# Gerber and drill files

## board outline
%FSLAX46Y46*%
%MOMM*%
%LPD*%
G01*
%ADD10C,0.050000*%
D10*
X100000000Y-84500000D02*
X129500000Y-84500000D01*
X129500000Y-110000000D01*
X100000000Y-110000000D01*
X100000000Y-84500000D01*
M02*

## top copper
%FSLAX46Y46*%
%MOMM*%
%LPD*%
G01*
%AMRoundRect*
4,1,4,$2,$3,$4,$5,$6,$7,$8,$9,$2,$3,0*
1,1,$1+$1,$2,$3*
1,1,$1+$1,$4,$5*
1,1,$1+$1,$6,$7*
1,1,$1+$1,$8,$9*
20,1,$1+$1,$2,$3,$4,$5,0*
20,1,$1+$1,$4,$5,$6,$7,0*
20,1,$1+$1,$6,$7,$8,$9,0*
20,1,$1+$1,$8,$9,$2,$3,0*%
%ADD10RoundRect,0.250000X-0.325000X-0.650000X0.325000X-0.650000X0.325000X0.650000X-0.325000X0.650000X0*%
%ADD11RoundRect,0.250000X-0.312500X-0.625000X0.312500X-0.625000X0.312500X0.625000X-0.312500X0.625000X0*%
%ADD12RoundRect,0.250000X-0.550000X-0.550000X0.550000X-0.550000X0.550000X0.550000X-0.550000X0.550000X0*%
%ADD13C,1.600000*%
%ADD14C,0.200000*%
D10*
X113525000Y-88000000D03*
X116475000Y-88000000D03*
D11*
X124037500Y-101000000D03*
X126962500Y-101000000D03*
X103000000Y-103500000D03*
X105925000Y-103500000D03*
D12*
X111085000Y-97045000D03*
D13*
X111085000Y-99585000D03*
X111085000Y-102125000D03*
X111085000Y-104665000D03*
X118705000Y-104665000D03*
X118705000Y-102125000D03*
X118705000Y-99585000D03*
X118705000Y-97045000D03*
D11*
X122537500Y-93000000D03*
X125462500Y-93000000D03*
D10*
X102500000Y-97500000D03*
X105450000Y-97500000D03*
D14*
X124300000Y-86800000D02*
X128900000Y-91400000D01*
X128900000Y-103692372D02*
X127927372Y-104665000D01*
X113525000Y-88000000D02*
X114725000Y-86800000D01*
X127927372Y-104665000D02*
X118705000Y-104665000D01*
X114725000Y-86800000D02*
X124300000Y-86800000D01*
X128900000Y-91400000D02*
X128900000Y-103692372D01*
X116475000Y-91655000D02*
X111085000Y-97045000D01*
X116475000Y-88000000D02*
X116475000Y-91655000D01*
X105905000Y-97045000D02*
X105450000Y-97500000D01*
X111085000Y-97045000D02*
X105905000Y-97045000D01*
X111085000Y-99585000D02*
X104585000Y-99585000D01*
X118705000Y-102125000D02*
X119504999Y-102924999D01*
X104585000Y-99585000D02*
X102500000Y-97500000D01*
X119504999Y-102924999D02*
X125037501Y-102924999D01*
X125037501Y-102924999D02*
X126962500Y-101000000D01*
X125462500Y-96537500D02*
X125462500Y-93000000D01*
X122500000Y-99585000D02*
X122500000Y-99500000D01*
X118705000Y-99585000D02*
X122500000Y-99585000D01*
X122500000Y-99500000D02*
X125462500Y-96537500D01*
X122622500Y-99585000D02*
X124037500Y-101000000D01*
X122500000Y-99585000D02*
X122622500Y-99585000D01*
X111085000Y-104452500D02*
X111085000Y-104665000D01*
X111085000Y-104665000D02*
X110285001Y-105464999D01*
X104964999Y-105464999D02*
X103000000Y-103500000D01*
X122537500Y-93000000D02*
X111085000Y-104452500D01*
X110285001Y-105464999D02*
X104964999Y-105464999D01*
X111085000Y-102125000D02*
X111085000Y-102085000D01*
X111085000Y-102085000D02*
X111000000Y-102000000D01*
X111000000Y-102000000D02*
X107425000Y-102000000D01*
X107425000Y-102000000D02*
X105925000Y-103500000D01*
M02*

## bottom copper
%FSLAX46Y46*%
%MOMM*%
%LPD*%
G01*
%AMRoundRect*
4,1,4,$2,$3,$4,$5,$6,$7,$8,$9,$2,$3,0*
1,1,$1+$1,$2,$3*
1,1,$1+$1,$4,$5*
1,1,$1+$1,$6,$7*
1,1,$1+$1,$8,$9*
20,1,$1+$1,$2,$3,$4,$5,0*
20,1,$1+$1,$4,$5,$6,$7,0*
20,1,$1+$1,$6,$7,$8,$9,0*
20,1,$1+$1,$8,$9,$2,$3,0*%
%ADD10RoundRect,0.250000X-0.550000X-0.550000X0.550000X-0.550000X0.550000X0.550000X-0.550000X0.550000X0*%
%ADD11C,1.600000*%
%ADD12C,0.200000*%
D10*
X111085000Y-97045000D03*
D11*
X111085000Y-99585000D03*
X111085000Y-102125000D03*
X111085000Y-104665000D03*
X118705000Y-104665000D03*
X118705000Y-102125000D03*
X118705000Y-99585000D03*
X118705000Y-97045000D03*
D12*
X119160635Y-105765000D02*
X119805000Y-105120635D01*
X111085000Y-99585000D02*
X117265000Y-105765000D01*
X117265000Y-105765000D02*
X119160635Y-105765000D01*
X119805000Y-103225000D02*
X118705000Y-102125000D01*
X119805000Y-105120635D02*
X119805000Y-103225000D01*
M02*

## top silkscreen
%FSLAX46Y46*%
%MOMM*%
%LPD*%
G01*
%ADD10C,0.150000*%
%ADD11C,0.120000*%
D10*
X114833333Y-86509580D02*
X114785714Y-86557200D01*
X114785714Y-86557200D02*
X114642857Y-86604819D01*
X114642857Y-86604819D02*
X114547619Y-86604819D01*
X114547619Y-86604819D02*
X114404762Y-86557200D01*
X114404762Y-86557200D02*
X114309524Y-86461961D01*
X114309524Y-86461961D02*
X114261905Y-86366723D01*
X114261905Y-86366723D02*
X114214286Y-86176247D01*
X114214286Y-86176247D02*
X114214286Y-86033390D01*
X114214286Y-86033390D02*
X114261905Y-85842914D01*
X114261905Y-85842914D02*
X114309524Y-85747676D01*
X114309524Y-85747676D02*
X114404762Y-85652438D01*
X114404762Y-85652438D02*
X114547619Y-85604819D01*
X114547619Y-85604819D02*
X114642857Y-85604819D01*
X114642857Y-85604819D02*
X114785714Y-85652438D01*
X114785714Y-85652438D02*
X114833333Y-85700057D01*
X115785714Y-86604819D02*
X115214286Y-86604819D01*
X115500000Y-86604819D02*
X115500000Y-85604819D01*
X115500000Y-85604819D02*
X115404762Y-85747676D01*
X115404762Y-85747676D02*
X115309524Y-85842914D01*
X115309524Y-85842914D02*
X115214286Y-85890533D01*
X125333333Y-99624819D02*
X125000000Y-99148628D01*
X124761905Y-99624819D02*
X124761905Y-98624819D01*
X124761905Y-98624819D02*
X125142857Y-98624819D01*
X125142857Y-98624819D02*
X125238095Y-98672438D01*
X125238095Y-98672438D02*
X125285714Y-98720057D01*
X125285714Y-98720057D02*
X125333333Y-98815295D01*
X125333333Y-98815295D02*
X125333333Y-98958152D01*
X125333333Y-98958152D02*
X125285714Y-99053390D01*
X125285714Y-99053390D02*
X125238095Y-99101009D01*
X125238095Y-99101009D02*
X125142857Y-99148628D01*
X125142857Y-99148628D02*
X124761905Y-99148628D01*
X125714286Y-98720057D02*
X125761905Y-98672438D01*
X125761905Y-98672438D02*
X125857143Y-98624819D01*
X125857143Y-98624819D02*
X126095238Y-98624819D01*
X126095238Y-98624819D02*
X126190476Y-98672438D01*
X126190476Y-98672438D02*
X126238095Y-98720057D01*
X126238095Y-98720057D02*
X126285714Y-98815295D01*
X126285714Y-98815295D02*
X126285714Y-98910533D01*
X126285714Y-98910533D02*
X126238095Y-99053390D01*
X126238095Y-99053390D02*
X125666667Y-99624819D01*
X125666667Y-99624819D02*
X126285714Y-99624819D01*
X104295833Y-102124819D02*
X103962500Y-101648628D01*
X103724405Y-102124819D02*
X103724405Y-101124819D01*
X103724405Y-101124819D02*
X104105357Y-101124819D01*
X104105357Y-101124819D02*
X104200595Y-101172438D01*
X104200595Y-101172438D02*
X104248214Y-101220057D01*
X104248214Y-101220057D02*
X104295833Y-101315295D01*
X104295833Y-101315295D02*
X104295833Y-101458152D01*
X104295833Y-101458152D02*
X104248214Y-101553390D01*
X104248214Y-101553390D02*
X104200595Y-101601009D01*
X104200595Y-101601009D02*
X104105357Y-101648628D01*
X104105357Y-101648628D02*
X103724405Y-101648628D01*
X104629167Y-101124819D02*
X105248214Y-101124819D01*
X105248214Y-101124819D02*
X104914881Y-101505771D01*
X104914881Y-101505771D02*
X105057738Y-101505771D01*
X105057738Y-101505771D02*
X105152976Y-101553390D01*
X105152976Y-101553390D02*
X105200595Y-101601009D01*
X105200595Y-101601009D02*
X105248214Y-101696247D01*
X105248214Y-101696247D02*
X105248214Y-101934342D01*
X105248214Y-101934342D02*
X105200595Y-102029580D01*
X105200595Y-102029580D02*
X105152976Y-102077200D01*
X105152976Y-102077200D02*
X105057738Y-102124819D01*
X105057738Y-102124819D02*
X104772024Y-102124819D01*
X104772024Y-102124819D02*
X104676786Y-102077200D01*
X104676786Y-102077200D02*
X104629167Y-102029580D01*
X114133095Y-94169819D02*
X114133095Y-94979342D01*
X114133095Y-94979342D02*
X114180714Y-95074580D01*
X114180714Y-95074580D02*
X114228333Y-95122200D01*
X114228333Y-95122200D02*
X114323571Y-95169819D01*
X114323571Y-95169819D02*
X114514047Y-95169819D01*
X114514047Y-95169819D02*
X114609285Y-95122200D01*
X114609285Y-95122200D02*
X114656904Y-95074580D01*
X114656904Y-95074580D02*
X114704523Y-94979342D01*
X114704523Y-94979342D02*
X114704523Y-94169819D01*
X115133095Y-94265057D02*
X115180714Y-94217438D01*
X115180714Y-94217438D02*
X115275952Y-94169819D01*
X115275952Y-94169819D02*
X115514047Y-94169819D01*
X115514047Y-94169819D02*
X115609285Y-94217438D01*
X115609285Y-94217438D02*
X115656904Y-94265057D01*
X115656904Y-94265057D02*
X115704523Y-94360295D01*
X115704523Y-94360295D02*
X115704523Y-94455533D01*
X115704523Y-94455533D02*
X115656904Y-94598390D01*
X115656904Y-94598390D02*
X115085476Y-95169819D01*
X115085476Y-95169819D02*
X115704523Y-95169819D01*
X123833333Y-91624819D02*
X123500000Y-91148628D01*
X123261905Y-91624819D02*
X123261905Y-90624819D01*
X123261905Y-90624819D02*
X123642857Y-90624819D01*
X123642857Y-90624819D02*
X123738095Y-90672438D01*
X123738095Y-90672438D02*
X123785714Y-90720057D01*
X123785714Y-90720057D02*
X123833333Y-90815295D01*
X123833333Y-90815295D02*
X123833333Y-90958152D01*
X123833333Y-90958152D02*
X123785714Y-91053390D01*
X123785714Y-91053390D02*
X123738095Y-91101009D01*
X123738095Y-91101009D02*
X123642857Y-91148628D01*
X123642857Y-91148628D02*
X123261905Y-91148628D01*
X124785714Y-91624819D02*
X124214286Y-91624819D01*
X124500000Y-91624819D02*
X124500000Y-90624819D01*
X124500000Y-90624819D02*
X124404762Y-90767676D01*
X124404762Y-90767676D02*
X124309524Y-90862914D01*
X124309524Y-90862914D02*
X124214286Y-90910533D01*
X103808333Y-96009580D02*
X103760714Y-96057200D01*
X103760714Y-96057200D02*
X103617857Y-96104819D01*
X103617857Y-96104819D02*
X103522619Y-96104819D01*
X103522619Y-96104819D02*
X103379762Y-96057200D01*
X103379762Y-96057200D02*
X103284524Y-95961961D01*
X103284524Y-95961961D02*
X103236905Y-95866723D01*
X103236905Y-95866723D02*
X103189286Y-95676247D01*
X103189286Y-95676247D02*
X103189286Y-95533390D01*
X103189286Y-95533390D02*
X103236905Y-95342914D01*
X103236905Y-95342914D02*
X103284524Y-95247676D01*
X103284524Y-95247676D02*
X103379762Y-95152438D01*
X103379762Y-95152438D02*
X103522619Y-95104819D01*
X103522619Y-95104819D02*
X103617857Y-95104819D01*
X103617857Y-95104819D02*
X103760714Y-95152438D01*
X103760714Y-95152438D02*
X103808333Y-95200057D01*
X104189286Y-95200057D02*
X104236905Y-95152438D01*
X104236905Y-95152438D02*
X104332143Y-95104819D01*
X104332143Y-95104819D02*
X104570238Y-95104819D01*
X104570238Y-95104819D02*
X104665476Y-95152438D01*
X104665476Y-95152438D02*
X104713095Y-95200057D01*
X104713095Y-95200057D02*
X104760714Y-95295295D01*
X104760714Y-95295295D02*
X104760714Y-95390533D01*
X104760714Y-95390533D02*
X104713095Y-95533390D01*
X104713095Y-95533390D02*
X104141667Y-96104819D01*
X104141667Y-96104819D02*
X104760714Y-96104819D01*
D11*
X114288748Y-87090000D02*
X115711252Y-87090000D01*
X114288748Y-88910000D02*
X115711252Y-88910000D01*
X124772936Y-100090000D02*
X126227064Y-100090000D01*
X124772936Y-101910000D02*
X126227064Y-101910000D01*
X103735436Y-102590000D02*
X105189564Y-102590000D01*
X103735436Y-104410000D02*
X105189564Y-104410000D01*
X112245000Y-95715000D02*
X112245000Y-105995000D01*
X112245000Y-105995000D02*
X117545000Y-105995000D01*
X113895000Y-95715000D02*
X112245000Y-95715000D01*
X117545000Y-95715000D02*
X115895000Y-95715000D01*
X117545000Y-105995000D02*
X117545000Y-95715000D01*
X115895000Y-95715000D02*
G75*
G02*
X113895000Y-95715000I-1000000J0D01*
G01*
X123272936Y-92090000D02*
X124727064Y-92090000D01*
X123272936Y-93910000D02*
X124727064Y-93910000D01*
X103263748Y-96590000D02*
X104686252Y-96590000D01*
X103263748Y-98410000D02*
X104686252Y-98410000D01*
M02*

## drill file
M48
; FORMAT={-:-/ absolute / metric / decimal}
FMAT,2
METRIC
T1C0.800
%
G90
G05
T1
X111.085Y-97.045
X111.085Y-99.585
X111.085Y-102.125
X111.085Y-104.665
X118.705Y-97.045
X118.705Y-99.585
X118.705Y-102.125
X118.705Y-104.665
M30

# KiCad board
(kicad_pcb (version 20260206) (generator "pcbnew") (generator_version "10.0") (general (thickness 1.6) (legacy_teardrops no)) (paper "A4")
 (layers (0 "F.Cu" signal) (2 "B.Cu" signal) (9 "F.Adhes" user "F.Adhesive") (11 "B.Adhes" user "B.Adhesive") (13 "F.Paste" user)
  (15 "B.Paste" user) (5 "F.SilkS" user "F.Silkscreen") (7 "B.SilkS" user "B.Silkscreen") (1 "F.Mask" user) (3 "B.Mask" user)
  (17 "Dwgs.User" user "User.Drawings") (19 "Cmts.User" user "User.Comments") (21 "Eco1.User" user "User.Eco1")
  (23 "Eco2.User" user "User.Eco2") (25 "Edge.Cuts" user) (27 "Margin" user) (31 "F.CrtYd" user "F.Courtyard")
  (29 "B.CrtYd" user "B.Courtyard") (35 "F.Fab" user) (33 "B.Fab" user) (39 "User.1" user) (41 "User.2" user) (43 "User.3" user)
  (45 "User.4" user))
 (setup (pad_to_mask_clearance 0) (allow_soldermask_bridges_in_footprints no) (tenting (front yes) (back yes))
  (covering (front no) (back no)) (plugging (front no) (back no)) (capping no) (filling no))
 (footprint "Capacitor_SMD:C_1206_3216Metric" (layer "F.Cu") (at 115 88)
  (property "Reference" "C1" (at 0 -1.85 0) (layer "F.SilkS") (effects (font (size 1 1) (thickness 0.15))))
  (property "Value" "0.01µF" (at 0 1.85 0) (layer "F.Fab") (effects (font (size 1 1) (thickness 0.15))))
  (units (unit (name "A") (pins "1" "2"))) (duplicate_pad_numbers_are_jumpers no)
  (fp_line (start -0.711252 -0.91) (end 0.711252 -0.91) (stroke (width 0.12) (type solid)) (layer "F.SilkS"))
  (fp_line (start -0.711252 0.91) (end 0.711252 0.91) (stroke (width 0.12) (type solid)) (layer "F.SilkS"))
  (pad "1" smd roundrect (at -1.475 0) (size 1.15 1.8) (layers "F.Cu" "F.Mask" "F.Paste") (roundrect_rratio 0.217391) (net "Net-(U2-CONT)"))
  (pad "2" smd roundrect (at 1.475 0) (size 1.15 1.8) (layers "F.Cu" "F.Mask" "F.Paste") (roundrect_rratio 0.217391) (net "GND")))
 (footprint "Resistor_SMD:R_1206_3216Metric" (layer "F.Cu") (at 125.5 101)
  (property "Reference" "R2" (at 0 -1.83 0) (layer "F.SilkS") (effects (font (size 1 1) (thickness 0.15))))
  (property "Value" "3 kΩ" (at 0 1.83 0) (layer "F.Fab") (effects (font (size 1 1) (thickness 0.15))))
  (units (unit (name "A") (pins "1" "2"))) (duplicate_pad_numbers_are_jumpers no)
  (fp_line (start -0.727064 -0.91) (end 0.727064 -0.91) (stroke (width 0.12) (type solid)) (layer "F.SilkS"))
  (fp_line (start -0.727064 0.91) (end 0.727064 0.91) (stroke (width 0.12) (type solid)) (layer "F.SilkS"))
  (pad "1" smd roundrect (at -1.4625 0) (size 1.125 1.75) (layers "F.Cu" "F.Mask" "F.Paste") (roundrect_rratio 0.222222)
   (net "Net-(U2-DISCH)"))
  (pad "2" smd roundrect (at 1.4625 0) (size 1.125 1.75) (layers "F.Cu" "F.Mask" "F.Paste") (roundrect_rratio 0.222222)
   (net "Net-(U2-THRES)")))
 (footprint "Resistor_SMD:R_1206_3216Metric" (layer "F.Cu") (at 104.4625 103.5)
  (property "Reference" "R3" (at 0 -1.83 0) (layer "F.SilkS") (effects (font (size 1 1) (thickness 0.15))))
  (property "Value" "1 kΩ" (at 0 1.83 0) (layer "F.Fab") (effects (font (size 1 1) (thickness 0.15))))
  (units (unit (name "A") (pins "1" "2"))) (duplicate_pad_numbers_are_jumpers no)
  (fp_line (start -0.727064 -0.91) (end 0.727064 -0.91) (stroke (width 0.12) (type solid)) (layer "F.SilkS"))
  (fp_line (start -0.727064 0.91) (end 0.727064 0.91) (stroke (width 0.12) (type solid)) (layer "F.SilkS"))
  (pad "1" smd roundrect (at -1.4625 0) (size 1.125 1.75) (layers "F.Cu" "F.Mask" "F.Paste") (roundrect_rratio 0.222222)
   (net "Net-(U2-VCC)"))
  (pad "2" smd roundrect (at 1.4625 0) (size 1.125 1.75) (layers "F.Cu" "F.Mask" "F.Paste") (roundrect_rratio 0.222222) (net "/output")))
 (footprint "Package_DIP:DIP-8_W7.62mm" (layer "F.Cu") (at 111.085 97.045)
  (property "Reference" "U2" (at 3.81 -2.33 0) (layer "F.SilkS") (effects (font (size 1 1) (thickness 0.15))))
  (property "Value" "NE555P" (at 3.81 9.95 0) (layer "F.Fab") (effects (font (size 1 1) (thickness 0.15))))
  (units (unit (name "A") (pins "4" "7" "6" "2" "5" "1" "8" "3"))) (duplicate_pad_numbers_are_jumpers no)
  (fp_line (start 1.16 -1.33) (end 1.16 8.95) (stroke (width 0.12) (type solid)) (layer "F.SilkS"))
  (fp_line (start 1.16 8.95) (end 6.46 8.95) (stroke (width 0.12) (type solid)) (layer "F.SilkS"))
  (fp_line (start 2.81 -1.33) (end 1.16 -1.33) (stroke (width 0.12) (type solid)) (layer "F.SilkS"))
  (fp_line (start 6.46 -1.33) (end 4.81 -1.33) (stroke (width 0.12) (type solid)) (layer "F.SilkS"))
  (fp_line (start 6.46 8.95) (end 6.46 -1.33) (stroke (width 0.12) (type solid)) (layer "F.SilkS"))
  (fp_arc (start 4.81 -1.33) (mid 3.81 -0.33) (end 2.81 -1.33) (stroke (width 0.12) (type solid)) (layer "F.SilkS"))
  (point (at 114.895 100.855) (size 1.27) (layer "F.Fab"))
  (pad "1" thru_hole roundrect (at 0 0) (size 1.6 1.6) (drill 0.8) (layers "*.Cu" "*.Mask") (remove_unused_layers no)
   (roundrect_rratio 0.15625) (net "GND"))
  (pad "2" thru_hole circle (at 0 2.54) (size 1.6 1.6) (drill 0.8) (layers "*.Cu" "*.Mask") (remove_unused_layers no) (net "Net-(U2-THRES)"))
  (pad "3" thru_hole circle (at 0 5.08) (size 1.6 1.6) (drill 0.8) (layers "*.Cu" "*.Mask") (remove_unused_layers no) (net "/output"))
  (pad "4" thru_hole circle (at 0 7.62) (size 1.6 1.6) (drill 0.8) (layers "*.Cu" "*.Mask") (remove_unused_layers no) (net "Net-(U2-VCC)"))
  (pad "5" thru_hole circle (at 7.62 7.62) (size 1.6 1.6) (drill 0.8) (layers "*.Cu" "*.Mask") (remove_unused_layers no)
   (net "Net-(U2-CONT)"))
  (pad "6" thru_hole circle (at 7.62 5.08) (size 1.6 1.6) (drill 0.8) (layers "*.Cu" "*.Mask") (remove_unused_layers no)
   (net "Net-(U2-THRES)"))
  (pad "7" thru_hole circle (at 7.62 2.54) (size 1.6 1.6) (drill 0.8) (layers "*.Cu" "*.Mask") (remove_unused_layers no)
   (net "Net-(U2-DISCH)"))
  (pad "8" thru_hole circle (at 7.62 0) (size 1.6 1.6) (drill 0.8) (layers "*.Cu" "*.Mask") (remove_unused_layers no) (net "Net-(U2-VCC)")))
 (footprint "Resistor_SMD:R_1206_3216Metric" (layer "F.Cu") (at 124 93)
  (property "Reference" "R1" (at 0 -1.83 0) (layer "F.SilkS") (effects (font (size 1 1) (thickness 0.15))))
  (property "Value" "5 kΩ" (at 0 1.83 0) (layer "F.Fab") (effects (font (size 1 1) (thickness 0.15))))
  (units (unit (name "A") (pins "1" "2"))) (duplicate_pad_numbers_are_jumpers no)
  (fp_line (start -0.727064 -0.91) (end 0.727064 -0.91) (stroke (width 0.12) (type solid)) (layer "F.SilkS"))
  (fp_line (start -0.727064 0.91) (end 0.727064 0.91) (stroke (width 0.12) (type solid)) (layer "F.SilkS"))
  (pad "1" smd roundrect (at -1.4625 0) (size 1.125 1.75) (layers "F.Cu" "F.Mask" "F.Paste") (roundrect_rratio 0.222222)
   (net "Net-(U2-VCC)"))
  (pad "2" smd roundrect (at 1.4625 0) (size 1.125 1.75) (layers "F.Cu" "F.Mask" "F.Paste") (roundrect_rratio 0.222222)
   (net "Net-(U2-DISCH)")))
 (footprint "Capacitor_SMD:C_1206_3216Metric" (layer "F.Cu") (at 103.975 97.5)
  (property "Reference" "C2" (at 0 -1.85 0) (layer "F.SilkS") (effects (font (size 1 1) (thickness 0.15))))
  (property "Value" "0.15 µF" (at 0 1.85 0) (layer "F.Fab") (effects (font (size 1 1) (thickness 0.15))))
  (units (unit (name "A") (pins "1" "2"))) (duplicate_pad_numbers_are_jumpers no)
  (fp_line (start -0.711252 -0.91) (end 0.711252 -0.91) (stroke (width 0.12) (type solid)) (layer "F.SilkS"))
  (fp_line (start -0.711252 0.91) (end 0.711252 0.91) (stroke (width 0.12) (type solid)) (layer "F.SilkS"))
  (pad "1" smd roundrect (at -1.475 0) (size 1.15 1.8) (layers "F.Cu" "F.Mask" "F.Paste") (roundrect_rratio 0.217391) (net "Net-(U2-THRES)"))
  (pad "2" smd roundrect (at 1.475 0) (size 1.15 1.8) (layers "F.Cu" "F.Mask" "F.Paste") (roundrect_rratio 0.217391) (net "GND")))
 (gr_rect (start 100 84.5) (end 129.5 110) (stroke (width 0.05) (type default)) (fill no) (layer "Edge.Cuts"))
 (segment (start 124.3 86.8) (end 128.9 91.4) (width 0.2) (layer "F.Cu") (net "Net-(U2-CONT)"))
 (segment (start 128.9 103.692372) (end 127.927372 104.665) (width 0.2) (layer "F.Cu") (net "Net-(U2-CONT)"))
 (segment (start 113.525 88) (end 114.725 86.8) (width 0.2) (layer "F.Cu") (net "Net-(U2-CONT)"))
 (segment (start 127.927372 104.665) (end 118.705 104.665) (width 0.2) (layer "F.Cu") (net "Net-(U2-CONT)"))
 (segment (start 114.725 86.8) (end 124.3 86.8) (width 0.2) (layer "F.Cu") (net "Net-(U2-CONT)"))
 (segment (start 128.9 91.4) (end 128.9 103.692372) (width 0.2) (layer "F.Cu") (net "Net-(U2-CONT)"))
 (segment (start 116.475 91.655) (end 111.085 97.045) (width 0.2) (layer "F.Cu") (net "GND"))
 (segment (start 116.475 88) (end 116.475 91.655) (width 0.2) (layer "F.Cu") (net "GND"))
 (segment (start 105.905 97.045) (end 105.45 97.5) (width 0.2) (layer "F.Cu") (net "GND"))
 (segment (start 111.085 97.045) (end 105.905 97.045) (width 0.2) (layer "F.Cu") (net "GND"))
 (segment (start 111.085 99.585) (end 104.585 99.585) (width 0.2) (layer "F.Cu") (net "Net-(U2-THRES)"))
 (segment (start 118.705 102.125) (end 119.504999 102.924999) (width 0.2) (layer "F.Cu") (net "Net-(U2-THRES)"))
 (segment (start 104.585 99.585) (end 102.5 97.5) (width 0.2) (layer "F.Cu") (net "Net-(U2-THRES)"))
 (segment (start 119.504999 102.924999) (end 125.037501 102.924999) (width 0.2) (layer "F.Cu") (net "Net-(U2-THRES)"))
 (segment (start 125.037501 102.924999) (end 126.9625 101) (width 0.2) (layer "F.Cu") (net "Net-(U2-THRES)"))
 (segment (start 119.160635 105.765) (end 119.805 105.120635) (width 0.2) (layer "B.Cu") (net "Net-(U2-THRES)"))
 (segment (start 111.085 99.585) (end 117.265 105.765) (width 0.2) (layer "B.Cu") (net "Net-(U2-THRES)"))
 (segment (start 117.265 105.765) (end 119.160635 105.765) (width 0.2) (layer "B.Cu") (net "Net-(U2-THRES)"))
 (segment (start 119.805 103.225) (end 118.705 102.125) (width 0.2) (layer "B.Cu") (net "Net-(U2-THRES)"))
 (segment (start 119.805 105.120635) (end 119.805 103.225) (width 0.2) (layer "B.Cu") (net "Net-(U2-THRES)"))
 (segment (start 125.4625 96.5375) (end 125.4625 93) (width 0.2) (layer "F.Cu") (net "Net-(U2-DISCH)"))
 (segment (start 122.5 99.585) (end 122.5 99.5) (width 0.2) (layer "F.Cu") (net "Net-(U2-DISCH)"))
 (segment (start 118.705 99.585) (end 122.5 99.585) (width 0.2) (layer "F.Cu") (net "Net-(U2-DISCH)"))
 (segment (start 122.5 99.5) (end 125.4625 96.5375) (width 0.2) (layer "F.Cu") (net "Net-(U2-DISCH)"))
 (segment (start 122.6225 99.585) (end 124.0375 101) (width 0.2) (layer "F.Cu") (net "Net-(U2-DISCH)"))
 (segment (start 122.5 99.585) (end 122.6225 99.585) (width 0.2) (layer "F.Cu") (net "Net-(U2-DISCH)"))
 (segment (start 111.085 104.4525) (end 111.085 104.665) (width 0.2) (layer "F.Cu") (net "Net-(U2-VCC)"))
 (segment (start 111.085 104.665) (end 110.285001 105.464999) (width 0.2) (layer "F.Cu") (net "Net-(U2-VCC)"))
 (segment (start 104.964999 105.464999) (end 103 103.5) (width 0.2) (layer "F.Cu") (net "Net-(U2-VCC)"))
 (segment (start 122.5375 93) (end 111.085 104.4525) (width 0.2) (layer "F.Cu") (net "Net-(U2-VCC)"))
 (segment (start 110.285001 105.464999) (end 104.964999 105.464999) (width 0.2) (layer "F.Cu") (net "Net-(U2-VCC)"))
 (segment (start 111.085 102.125) (end 111.085 102.085) (width 0.2) (layer "F.Cu") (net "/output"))
 (segment (start 111.085 102.085) (end 111 102) (width 0.2) (layer "F.Cu") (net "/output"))
 (segment (start 111 102) (end 107.425 102) (width 0.2) (layer "F.Cu") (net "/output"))
 (segment (start 107.425 102) (end 105.925 103.5) (width 0.2) (layer "F.Cu") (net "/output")))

